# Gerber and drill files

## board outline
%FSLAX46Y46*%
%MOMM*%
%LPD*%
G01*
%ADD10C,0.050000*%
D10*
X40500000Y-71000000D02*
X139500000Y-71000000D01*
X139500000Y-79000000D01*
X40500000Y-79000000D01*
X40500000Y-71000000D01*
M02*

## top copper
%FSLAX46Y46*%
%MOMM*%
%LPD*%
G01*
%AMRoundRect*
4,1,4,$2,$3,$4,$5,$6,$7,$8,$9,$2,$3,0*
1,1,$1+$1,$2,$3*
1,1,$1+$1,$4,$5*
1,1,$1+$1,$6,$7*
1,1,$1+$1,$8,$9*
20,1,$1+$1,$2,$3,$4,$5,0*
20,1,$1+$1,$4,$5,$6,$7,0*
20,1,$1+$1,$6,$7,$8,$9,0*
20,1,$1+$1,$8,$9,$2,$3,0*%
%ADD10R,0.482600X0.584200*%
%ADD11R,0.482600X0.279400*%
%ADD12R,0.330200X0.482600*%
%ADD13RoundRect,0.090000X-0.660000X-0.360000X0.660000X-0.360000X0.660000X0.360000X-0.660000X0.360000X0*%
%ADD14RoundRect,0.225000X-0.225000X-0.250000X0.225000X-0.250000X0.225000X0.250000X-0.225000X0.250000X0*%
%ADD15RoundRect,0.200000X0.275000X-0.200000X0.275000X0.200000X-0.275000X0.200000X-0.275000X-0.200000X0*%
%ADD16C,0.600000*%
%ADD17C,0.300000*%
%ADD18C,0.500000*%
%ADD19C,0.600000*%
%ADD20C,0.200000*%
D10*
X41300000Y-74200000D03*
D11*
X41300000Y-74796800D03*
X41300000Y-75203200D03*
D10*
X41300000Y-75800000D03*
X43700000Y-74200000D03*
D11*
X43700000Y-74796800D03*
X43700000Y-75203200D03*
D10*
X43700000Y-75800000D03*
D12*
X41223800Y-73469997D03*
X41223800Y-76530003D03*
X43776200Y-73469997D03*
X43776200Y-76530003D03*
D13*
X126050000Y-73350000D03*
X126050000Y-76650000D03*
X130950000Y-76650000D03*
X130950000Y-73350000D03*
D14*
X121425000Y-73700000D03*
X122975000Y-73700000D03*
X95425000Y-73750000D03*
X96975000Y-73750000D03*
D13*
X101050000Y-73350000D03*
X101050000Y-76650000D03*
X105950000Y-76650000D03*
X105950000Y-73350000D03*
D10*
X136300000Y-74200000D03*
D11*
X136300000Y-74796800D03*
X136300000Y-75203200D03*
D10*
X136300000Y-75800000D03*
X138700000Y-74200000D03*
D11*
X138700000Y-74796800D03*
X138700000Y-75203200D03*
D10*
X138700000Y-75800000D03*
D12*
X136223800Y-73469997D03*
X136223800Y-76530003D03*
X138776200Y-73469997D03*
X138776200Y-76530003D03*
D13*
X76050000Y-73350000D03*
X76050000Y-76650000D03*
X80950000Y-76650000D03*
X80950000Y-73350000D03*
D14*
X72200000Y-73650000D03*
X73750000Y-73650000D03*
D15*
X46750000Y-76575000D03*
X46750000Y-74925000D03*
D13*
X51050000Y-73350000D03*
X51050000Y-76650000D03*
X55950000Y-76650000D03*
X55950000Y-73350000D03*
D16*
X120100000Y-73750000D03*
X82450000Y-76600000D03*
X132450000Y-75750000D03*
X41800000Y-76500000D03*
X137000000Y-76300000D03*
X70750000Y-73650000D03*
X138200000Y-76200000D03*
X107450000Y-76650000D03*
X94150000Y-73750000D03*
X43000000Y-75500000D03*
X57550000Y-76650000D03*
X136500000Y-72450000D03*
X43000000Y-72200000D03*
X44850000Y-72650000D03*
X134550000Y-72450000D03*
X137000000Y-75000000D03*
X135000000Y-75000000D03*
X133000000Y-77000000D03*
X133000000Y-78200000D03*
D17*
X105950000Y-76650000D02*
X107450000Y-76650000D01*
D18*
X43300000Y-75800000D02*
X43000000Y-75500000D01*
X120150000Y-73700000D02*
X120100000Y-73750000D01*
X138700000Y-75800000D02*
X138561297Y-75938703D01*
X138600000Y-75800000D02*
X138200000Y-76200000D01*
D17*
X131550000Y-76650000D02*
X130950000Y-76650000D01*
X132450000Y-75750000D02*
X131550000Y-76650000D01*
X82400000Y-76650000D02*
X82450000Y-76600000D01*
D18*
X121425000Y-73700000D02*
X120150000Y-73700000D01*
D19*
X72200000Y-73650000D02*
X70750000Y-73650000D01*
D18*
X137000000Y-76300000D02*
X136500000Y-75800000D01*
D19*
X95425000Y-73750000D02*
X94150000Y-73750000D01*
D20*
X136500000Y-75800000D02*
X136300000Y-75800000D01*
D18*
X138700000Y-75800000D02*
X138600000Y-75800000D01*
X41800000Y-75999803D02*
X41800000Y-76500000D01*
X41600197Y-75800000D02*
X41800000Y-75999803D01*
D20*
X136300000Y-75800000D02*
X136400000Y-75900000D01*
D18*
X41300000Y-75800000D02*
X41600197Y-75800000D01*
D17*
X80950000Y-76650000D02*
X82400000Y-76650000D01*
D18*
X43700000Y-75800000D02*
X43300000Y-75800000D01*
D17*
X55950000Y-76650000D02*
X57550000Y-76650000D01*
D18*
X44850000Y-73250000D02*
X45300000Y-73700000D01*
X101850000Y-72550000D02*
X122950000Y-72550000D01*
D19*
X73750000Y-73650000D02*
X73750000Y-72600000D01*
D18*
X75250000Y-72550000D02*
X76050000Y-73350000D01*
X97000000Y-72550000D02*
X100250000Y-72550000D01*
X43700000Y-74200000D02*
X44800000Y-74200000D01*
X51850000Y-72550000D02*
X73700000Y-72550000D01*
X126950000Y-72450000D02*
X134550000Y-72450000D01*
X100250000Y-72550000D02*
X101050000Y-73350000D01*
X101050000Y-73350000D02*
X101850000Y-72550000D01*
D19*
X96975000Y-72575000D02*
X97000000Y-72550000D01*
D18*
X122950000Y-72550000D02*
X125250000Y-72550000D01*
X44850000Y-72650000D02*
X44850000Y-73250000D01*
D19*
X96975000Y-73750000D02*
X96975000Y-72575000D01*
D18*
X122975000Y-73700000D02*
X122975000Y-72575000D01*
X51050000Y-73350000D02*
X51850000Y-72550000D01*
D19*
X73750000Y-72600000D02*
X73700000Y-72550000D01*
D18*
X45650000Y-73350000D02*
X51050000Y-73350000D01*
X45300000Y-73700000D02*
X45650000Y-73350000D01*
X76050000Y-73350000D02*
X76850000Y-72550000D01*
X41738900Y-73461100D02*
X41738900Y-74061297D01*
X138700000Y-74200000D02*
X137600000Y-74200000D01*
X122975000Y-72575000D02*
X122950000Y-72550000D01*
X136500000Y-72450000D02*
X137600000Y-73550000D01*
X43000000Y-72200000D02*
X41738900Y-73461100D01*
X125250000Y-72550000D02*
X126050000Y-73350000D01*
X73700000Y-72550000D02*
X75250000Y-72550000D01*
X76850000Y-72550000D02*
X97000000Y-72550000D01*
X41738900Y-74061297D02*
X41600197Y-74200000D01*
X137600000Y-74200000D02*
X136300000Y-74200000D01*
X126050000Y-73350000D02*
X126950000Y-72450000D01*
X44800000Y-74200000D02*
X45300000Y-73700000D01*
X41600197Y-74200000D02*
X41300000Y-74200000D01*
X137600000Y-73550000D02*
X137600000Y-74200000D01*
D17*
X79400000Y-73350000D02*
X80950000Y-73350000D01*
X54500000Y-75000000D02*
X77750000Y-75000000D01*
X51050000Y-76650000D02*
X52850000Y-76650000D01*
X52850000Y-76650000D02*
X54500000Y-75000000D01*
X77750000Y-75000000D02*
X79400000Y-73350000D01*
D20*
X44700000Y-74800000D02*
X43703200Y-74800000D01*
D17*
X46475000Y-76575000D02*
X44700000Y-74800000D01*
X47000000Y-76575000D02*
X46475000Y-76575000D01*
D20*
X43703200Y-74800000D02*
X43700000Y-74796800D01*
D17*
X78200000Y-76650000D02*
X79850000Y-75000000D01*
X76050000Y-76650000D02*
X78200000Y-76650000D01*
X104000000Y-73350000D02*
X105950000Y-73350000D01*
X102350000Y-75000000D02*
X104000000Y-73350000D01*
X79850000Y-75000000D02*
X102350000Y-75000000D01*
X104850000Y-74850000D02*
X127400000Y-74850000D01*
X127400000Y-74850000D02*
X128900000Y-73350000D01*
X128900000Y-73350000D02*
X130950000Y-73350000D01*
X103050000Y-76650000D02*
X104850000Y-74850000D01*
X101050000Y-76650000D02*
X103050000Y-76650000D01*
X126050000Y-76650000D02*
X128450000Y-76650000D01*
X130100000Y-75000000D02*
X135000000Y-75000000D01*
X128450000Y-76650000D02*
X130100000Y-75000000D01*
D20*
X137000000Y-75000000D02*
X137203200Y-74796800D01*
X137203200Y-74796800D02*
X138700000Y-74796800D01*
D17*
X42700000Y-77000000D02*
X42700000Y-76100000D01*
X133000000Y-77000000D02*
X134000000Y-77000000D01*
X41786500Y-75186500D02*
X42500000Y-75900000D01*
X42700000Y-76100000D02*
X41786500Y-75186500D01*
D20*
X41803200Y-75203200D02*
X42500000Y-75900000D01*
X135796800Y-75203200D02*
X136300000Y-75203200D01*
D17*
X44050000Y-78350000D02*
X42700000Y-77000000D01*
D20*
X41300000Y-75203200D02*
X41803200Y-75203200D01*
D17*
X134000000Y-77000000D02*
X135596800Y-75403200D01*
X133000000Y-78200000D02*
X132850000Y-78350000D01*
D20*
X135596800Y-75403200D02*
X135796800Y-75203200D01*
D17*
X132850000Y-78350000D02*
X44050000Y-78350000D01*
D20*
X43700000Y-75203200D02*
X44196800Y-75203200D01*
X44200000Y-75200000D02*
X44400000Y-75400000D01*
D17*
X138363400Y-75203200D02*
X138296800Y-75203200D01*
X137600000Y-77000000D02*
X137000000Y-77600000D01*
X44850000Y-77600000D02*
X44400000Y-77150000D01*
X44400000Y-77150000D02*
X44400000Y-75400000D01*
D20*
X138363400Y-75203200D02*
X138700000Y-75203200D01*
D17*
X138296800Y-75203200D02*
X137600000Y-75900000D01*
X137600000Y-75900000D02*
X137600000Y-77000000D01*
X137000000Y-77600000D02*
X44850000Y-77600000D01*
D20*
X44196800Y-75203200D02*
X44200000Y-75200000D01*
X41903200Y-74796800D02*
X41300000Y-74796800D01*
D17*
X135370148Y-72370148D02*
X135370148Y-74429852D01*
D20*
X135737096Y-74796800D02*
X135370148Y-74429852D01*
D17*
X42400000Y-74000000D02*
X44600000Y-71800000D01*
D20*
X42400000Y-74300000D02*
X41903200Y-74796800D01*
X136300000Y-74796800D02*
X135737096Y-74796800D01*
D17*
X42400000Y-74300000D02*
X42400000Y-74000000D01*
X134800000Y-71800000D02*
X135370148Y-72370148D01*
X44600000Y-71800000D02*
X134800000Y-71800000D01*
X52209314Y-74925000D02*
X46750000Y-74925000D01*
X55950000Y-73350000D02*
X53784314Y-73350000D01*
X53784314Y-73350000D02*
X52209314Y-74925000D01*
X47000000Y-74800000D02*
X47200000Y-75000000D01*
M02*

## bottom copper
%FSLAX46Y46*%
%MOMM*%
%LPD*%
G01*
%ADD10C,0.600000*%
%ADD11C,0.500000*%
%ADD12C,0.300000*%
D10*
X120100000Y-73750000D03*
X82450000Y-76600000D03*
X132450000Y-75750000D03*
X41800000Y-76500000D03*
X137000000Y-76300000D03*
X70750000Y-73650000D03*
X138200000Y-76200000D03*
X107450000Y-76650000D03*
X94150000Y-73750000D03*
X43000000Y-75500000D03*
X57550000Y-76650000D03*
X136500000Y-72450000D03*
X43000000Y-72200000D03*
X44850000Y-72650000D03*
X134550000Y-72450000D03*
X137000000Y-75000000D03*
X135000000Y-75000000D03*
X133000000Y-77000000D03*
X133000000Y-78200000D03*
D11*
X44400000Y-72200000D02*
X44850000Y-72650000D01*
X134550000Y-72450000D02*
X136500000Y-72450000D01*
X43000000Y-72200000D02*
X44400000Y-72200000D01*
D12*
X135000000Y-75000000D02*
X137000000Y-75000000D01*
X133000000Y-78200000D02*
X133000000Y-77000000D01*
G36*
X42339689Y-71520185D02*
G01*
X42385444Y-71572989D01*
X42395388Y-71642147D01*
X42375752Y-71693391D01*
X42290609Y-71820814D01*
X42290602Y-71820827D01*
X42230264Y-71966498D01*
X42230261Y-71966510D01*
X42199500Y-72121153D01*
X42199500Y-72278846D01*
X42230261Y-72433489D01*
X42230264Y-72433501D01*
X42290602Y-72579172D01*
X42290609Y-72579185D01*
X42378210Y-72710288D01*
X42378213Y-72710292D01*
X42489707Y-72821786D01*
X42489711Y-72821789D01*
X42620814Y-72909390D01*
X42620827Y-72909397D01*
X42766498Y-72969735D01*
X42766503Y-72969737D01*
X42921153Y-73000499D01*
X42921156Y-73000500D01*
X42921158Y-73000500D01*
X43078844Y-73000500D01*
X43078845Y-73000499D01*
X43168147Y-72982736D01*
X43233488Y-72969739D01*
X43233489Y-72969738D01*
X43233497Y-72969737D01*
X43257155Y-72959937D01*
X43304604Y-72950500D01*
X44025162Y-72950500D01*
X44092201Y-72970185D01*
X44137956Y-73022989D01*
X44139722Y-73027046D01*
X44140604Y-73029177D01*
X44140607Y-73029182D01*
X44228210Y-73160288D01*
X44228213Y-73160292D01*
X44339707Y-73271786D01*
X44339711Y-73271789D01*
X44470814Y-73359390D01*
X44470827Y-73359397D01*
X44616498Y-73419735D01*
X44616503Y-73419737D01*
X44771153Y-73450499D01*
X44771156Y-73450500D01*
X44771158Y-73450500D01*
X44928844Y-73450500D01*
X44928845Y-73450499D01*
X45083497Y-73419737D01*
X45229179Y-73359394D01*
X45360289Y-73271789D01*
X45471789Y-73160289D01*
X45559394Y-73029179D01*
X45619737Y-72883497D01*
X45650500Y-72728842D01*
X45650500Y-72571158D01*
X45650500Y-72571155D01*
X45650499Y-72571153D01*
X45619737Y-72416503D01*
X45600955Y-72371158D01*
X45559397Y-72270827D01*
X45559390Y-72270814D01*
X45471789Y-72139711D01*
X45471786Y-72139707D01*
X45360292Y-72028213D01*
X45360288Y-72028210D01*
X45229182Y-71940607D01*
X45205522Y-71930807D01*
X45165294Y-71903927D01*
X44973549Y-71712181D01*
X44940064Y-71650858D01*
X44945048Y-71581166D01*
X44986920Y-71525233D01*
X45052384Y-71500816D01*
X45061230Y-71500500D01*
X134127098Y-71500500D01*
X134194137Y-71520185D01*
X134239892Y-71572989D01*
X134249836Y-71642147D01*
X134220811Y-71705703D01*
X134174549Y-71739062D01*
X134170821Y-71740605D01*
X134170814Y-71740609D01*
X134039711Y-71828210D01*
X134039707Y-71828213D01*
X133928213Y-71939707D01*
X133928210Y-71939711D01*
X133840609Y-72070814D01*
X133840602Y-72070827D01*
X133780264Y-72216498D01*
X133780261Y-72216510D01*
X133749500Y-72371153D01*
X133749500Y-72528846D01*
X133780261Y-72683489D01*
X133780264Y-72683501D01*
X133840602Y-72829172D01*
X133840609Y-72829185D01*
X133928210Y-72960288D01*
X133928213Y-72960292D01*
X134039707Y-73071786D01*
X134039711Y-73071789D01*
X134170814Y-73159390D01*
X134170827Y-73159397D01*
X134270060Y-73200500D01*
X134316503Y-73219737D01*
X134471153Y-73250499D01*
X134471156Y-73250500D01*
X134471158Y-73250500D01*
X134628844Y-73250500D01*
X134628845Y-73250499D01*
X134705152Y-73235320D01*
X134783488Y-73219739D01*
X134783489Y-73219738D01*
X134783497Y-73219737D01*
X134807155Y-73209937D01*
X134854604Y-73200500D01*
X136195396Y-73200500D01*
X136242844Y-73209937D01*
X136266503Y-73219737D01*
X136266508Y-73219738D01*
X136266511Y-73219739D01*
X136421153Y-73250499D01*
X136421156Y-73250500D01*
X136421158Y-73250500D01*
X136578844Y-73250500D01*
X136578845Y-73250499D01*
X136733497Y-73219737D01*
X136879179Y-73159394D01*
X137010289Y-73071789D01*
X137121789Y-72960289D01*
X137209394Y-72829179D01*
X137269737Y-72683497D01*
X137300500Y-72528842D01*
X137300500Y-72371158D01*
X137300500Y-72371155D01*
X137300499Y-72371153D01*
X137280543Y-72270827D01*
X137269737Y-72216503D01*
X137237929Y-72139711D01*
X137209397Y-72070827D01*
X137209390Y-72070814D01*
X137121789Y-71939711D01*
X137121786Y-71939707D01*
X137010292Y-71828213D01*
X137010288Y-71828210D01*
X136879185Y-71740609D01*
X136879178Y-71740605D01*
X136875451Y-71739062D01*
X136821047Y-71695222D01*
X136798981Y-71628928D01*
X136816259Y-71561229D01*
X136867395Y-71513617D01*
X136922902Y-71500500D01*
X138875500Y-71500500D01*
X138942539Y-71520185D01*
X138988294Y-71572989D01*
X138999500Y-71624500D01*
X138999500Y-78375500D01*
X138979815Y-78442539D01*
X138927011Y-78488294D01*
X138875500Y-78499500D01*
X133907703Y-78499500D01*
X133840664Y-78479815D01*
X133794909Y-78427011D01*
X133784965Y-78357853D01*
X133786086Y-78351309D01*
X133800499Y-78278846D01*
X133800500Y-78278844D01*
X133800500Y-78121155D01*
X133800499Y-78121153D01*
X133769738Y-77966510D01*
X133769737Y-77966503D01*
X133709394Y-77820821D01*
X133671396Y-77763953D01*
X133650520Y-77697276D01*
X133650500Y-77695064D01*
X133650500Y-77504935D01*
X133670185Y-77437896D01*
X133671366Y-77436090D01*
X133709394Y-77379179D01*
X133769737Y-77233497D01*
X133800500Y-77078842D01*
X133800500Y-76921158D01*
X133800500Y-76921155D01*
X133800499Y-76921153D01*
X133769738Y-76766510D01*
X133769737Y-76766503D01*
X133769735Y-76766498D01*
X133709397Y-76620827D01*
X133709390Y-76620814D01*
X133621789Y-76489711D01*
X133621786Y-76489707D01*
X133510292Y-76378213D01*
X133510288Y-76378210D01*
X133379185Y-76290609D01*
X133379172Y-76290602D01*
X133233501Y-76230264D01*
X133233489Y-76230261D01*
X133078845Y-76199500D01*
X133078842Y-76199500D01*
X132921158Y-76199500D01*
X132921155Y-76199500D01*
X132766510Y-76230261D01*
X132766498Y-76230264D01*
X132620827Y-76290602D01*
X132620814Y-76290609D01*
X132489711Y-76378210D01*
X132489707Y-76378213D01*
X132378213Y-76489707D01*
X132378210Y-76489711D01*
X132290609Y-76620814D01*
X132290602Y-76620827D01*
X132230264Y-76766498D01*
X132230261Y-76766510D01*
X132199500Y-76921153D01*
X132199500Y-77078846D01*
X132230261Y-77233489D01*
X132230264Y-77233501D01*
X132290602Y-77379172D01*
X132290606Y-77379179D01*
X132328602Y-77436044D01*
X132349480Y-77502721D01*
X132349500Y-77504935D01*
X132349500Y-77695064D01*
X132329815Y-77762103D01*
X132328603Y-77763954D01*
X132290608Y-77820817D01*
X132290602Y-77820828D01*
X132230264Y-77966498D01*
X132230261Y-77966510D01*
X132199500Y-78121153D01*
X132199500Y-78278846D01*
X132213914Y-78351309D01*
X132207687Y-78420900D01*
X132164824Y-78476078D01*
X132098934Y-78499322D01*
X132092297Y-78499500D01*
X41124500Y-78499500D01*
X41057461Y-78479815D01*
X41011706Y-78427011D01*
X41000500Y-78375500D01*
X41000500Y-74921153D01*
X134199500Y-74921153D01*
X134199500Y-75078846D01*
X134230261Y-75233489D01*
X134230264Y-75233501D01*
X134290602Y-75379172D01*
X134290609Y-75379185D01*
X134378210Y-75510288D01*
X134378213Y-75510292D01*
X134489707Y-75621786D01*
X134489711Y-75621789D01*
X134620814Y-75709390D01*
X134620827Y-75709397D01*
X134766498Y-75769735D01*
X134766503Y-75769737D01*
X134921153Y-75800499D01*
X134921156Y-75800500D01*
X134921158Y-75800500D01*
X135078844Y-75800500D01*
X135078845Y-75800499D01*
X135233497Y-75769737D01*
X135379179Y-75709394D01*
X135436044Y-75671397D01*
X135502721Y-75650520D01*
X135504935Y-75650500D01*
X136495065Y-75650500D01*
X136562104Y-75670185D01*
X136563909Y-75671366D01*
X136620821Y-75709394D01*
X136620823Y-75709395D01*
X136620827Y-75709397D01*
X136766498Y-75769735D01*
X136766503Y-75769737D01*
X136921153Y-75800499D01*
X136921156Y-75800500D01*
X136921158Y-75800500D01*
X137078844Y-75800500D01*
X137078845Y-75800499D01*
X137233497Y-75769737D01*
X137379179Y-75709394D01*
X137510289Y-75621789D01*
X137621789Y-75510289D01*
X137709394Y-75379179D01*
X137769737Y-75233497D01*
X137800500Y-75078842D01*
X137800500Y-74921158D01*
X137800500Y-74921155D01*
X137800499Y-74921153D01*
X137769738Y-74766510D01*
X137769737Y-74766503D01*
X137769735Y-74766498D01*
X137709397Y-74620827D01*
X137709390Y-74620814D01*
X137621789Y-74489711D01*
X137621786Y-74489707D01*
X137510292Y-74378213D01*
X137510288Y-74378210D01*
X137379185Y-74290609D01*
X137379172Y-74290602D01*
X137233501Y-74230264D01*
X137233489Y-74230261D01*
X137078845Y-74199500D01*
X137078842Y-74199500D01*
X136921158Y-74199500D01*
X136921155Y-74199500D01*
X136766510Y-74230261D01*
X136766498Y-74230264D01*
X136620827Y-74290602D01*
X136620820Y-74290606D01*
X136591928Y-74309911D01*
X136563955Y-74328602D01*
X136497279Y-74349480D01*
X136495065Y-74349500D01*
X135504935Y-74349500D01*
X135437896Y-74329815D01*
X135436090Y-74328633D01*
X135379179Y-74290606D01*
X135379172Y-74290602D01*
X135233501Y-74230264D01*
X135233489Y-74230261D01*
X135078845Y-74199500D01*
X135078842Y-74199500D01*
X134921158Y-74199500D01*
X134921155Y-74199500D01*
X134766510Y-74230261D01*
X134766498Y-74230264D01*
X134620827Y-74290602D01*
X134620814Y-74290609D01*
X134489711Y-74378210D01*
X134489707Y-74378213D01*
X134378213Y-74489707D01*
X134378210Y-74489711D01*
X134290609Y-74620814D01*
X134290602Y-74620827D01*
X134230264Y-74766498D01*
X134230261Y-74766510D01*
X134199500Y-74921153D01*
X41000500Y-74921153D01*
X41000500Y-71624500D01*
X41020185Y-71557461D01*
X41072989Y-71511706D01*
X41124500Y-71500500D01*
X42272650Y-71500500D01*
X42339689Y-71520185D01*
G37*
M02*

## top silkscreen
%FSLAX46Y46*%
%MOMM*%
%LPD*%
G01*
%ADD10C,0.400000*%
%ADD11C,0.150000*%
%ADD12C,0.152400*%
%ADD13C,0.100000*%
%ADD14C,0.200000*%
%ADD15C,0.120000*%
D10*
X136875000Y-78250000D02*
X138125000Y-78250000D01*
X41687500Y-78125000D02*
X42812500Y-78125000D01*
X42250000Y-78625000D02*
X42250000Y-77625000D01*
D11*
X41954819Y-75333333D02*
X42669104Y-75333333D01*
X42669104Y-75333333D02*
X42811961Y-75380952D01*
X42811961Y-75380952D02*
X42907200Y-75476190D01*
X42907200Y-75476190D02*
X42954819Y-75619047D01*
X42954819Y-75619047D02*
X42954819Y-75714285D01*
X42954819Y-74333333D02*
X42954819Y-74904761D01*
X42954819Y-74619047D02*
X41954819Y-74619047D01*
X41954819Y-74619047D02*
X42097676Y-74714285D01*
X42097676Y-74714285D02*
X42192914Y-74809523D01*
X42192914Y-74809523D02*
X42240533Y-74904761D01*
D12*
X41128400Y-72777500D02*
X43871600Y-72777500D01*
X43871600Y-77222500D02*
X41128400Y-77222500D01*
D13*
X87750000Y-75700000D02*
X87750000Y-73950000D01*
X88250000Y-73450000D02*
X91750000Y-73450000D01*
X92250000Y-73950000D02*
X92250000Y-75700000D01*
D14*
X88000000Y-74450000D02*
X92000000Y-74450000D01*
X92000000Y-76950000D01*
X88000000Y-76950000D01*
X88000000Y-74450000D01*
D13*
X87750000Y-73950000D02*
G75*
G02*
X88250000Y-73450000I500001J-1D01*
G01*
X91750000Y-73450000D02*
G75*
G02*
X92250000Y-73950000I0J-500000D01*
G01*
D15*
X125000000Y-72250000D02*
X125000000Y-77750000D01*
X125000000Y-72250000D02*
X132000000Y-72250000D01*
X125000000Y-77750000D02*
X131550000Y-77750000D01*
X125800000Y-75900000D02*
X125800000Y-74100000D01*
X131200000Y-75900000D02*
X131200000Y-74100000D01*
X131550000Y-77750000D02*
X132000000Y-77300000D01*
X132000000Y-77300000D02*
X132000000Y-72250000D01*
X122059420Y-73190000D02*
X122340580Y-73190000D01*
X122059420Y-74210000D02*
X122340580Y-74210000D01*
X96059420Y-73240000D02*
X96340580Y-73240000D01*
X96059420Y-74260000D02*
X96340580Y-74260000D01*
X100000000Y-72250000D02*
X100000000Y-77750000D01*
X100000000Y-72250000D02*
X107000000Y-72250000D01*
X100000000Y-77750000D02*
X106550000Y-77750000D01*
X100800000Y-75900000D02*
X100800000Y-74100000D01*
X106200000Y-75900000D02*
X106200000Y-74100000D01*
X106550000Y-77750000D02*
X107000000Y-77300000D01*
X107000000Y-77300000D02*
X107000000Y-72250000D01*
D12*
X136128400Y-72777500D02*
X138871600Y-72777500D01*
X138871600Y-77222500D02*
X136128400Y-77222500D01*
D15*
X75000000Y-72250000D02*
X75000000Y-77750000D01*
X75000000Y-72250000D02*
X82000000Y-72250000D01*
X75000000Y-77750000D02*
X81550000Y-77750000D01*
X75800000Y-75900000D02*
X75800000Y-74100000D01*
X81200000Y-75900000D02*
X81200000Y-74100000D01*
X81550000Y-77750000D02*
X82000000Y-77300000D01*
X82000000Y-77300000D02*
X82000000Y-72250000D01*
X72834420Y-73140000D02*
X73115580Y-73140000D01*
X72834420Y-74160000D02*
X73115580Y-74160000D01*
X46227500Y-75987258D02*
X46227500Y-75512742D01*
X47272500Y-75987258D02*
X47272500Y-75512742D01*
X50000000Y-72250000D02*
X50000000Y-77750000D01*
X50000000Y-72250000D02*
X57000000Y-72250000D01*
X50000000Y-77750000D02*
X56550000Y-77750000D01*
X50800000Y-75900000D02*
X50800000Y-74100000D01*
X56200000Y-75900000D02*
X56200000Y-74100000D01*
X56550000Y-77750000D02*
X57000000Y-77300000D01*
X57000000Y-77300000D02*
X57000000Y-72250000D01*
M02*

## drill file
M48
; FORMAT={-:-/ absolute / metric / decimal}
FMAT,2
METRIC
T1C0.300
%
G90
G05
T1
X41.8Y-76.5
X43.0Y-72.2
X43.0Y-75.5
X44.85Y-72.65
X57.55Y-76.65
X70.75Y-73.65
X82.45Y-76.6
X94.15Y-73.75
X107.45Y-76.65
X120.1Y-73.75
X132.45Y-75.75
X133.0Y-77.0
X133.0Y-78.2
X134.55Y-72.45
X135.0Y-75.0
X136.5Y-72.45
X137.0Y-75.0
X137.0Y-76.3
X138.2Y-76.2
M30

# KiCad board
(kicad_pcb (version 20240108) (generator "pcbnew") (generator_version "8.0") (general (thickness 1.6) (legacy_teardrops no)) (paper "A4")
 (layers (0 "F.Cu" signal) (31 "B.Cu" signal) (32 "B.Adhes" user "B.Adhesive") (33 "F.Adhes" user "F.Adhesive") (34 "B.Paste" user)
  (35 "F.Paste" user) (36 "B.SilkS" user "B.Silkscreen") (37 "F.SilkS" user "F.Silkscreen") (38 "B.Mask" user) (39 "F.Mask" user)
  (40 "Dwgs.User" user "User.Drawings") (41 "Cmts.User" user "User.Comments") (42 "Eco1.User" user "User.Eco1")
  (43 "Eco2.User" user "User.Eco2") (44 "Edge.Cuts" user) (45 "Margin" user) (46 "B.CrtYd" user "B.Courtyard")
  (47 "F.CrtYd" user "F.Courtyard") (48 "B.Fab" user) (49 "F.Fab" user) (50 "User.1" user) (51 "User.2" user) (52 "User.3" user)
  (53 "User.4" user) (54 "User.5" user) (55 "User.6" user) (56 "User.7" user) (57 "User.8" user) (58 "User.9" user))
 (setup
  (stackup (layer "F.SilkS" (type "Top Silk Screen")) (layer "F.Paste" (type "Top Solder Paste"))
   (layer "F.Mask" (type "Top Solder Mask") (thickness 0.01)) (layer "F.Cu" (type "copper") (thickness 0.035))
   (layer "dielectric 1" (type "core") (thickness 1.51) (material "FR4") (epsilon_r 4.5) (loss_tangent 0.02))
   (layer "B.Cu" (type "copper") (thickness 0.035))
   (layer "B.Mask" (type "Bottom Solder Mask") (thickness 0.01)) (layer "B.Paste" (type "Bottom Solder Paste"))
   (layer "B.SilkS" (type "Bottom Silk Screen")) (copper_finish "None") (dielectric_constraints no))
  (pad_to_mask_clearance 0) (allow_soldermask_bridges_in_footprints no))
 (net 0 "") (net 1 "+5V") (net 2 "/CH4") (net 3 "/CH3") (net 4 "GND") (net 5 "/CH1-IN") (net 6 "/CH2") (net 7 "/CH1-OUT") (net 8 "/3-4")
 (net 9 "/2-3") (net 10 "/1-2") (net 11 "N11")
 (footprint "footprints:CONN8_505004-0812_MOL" (layer "F.Cu") (at 42.5 75 90)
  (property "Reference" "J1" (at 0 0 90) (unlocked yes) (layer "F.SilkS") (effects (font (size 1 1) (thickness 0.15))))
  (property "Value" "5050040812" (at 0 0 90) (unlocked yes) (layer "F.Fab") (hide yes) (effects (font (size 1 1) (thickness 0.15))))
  (fp_line (start 2.2225 -1.3716) (end 2.2225 1.3716) (stroke (width 0.1524) (type solid)) (layer "F.SilkS"))
  (fp_line (start -2.2225 1.3716) (end -2.2225 -1.3716) (stroke (width 0.1524) (type solid)) (layer "F.SilkS"))
  (pad "1" smd rect (at 0.8 -1.2 90) (size 0.5842 0.4826) (layers "F.Cu" "F.Paste" "F.Mask") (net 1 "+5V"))
  (pad "2" smd rect (at 0.2032 -1.2 90) (size 0.2794 0.4826) (layers "F.Cu" "F.Paste" "F.Mask") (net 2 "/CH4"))
  (pad "3" smd rect (at -0.2032 -1.2 90) (size 0.2794 0.4826) (layers "F.Cu" "F.Paste" "F.Mask") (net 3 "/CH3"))
  (pad "4" smd rect (at -0.8 -1.2 90) (size 0.5842 0.4826) (layers "F.Cu" "F.Paste" "F.Mask") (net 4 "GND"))
  (pad "5" smd rect (at 0.8 1.2 90) (size 0.5842 0.4826) (layers "F.Cu" "F.Paste" "F.Mask") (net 1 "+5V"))
  (pad "6" smd rect (at 0.2032 1.2 90) (size 0.2794 0.4826) (layers "F.Cu" "F.Paste" "F.Mask") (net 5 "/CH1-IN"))
  (pad "7" smd rect (at -0.2032 1.2 90) (size 0.2794 0.4826) (layers "F.Cu" "F.Paste" "F.Mask") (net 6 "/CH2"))
  (pad "8" smd rect (at -0.8 1.2 90) (size 0.5842 0.4826) (layers "F.Cu" "F.Paste" "F.Mask") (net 4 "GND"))
  (pad "9" smd rect (at 1.530003 -1.2762 90) (size 0.4826 0.3302) (layers "F.Cu" "F.Paste" "F.Mask"))
  (pad "10" smd rect (at -1.530003 -1.2762 90) (size 0.4826 0.3302) (layers "F.Cu" "F.Paste" "F.Mask"))
  (pad "11" smd rect (at 1.530003 1.2762 90) (size 0.4826 0.3302) (layers "F.Cu" "F.Paste" "F.Mask"))
  (pad "12" smd rect (at -1.530003 1.2762 90) (size 0.4826 0.3302) (layers "F.Cu" "F.Paste" "F.Mask")))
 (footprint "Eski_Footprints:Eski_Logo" (layer "F.Cu") (at 90 76.95)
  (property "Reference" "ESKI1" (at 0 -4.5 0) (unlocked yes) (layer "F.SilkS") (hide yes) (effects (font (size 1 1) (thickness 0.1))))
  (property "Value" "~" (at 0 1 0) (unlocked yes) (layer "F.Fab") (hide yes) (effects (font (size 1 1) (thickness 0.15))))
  (fp_line (start -2.25 -1.25) (end -2.25 -3) (stroke (width 0.1) (type default)) (layer "F.SilkS"))
  (fp_line (start -1.75 -3.5) (end 1.75 -3.5) (stroke (width 0.1) (type default)) (layer "F.SilkS"))
  (fp_line (start 2.25 -3) (end 2.25 -1.25) (stroke (width 0.1) (type default)) (layer "F.SilkS"))
  (fp_rect (start -2 -2.5) (end 2 0) (stroke (width 0.2) (type default)) (fill none) (layer "F.SilkS"))
  (fp_arc (start -2.25 -3) (mid -2.103553 -3.353553) (end -1.75 -3.5) (stroke (width 0.1) (type default)) (layer "F.SilkS"))
  (fp_arc (start 1.75 -3.5) (mid 2.103553 -3.353553) (end 2.25 -3) (stroke (width 0.1) (type default)) (layer "F.SilkS")))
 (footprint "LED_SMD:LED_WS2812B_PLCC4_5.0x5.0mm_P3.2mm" (layer "F.Cu") (at 128.5 75)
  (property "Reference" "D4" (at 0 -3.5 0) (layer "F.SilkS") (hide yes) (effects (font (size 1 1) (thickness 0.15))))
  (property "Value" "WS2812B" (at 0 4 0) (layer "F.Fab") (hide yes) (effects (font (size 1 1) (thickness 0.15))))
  (fp_line (start -3.5 -2.75) (end -3.5 2.75) (stroke (width 0.12) (type default)) (layer "F.SilkS"))
  (fp_line (start -3.5 -2.75) (end 3.5 -2.75) (stroke (width 0.12) (type solid)) (layer "F.SilkS"))
  (fp_line (start -3.5 2.75) (end 3.05 2.75) (stroke (width 0.12) (type solid)) (layer "F.SilkS"))
  (fp_line (start -2.7 0.9) (end -2.7 -0.9) (stroke (width 0.12) (type default)) (layer "F.SilkS"))
  (fp_line (start 2.7 0.9) (end 2.7 -0.9) (stroke (width 0.12) (type default)) (layer "F.SilkS"))
  (fp_line (start 3.05 2.75) (end 3.5 2.3) (stroke (width 0.12) (type default)) (layer "F.SilkS"))
  (fp_line (start 3.5 2.3) (end 3.5 -2.75) (stroke (width 0.12) (type default)) (layer "F.SilkS"))
  (pad "1" smd roundrect (at -2.45 -1.65) (size 1.5 0.9) (layers "F.Cu" "F.Paste" "F.Mask") (roundrect_rratio 0.1) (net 1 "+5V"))
  (pad "2" smd roundrect (at -2.45 1.65) (size 1.5 0.9) (layers "F.Cu" "F.Paste" "F.Mask") (roundrect_rratio 0.1) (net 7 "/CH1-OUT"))
  (pad "3" smd roundrect (at 2.45 1.65) (size 1.5 0.9) (layers "F.Cu" "F.Paste" "F.Mask") (roundrect_rratio 0.1) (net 4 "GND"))
  (pad "4" smd roundrect (at 2.45 -1.65) (size 1.5 0.9) (layers "F.Cu" "F.Paste" "F.Mask") (roundrect_rratio 0.1) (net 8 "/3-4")))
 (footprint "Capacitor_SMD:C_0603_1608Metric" (layer "F.Cu") (at 122.2 73.7)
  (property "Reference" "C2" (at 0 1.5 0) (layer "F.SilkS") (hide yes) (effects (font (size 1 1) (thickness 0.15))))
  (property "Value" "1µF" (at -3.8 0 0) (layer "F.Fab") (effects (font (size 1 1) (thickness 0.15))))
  (fp_line (start -0.14058 -0.51) (end 0.14058 -0.51) (stroke (width 0.12) (type solid)) (layer "F.SilkS"))
  (fp_line (start -0.14058 0.51) (end 0.14058 0.51) (stroke (width 0.12) (type solid)) (layer "F.SilkS"))
  (pad "1" smd roundrect (at -0.775 0) (size 0.9 0.95) (layers "F.Cu" "F.Paste" "F.Mask") (roundrect_rratio 0.25) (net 4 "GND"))
  (pad "2" smd roundrect (at 0.775 0) (size 0.9 0.95) (layers "F.Cu" "F.Paste" "F.Mask") (roundrect_rratio 0.25) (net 1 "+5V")))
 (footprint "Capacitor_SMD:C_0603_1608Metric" (layer "F.Cu") (at 96.2 73.75)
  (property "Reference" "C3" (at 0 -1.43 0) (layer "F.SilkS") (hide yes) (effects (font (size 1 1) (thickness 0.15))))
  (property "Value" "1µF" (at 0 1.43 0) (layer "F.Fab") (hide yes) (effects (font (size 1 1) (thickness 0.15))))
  (fp_line (start -0.14058 -0.51) (end 0.14058 -0.51) (stroke (width 0.12) (type solid)) (layer "F.SilkS"))
  (fp_line (start -0.14058 0.51) (end 0.14058 0.51) (stroke (width 0.12) (type solid)) (layer "F.SilkS"))
  (pad "1" smd roundrect (at -0.775 0) (size 0.9 0.95) (layers "F.Cu" "F.Paste" "F.Mask") (roundrect_rratio 0.25) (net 4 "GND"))
  (pad "2" smd roundrect (at 0.775 0) (size 0.9 0.95) (layers "F.Cu" "F.Paste" "F.Mask") (roundrect_rratio 0.25) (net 1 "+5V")))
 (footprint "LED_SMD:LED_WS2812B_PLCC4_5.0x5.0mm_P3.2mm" (layer "F.Cu") (at 103.5 75)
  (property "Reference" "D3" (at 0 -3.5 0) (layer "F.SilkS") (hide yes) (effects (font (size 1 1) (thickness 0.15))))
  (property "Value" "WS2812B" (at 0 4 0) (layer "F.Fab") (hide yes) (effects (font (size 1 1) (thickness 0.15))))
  (fp_line (start -3.5 -2.75) (end -3.5 2.75) (stroke (width 0.12) (type default)) (layer "F.SilkS"))
  (fp_line (start -3.5 -2.75) (end 3.5 -2.75) (stroke (width 0.12) (type solid)) (layer "F.SilkS"))
  (fp_line (start -3.5 2.75) (end 3.05 2.75) (stroke (width 0.12) (type solid)) (layer "F.SilkS"))
  (fp_line (start -2.7 0.9) (end -2.7 -0.9) (stroke (width 0.12) (type default)) (layer "F.SilkS"))
  (fp_line (start 2.7 0.9) (end 2.7 -0.9) (stroke (width 0.12) (type default)) (layer "F.SilkS"))
  (fp_line (start 3.05 2.75) (end 3.5 2.3) (stroke (width 0.12) (type default)) (layer "F.SilkS"))
  (fp_line (start 3.5 2.3) (end 3.5 -2.75) (stroke (width 0.12) (type default)) (layer "F.SilkS"))
  (pad "1" smd roundrect (at -2.45 -1.65) (size 1.5 0.9) (layers "F.Cu" "F.Paste" "F.Mask") (roundrect_rratio 0.1) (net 1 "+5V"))
  (pad "2" smd roundrect (at -2.45 1.65) (size 1.5 0.9) (layers "F.Cu" "F.Paste" "F.Mask") (roundrect_rratio 0.1) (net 8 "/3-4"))
  (pad "3" smd roundrect (at 2.45 1.65) (size 1.5 0.9) (layers "F.Cu" "F.Paste" "F.Mask") (roundrect_rratio 0.1) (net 4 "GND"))
  (pad "4" smd roundrect (at 2.45 -1.65) (size 1.5 0.9) (layers "F.Cu" "F.Paste" "F.Mask") (roundrect_rratio 0.1) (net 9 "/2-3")))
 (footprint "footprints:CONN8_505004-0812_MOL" (layer "F.Cu") (at 137.5 75 90)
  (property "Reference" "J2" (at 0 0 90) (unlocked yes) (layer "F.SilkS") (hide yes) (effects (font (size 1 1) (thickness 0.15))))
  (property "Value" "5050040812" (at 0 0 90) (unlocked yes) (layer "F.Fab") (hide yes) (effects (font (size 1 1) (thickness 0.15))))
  (fp_line (start 2.2225 -1.3716) (end 2.2225 1.3716) (stroke (width 0.1524) (type solid)) (layer "F.SilkS"))
  (fp_line (start -2.2225 1.3716) (end -2.2225 -1.3716) (stroke (width 0.1524) (type solid)) (layer "F.SilkS"))
  (pad "1" smd rect (at 0.8 -1.2 90) (size 0.5842 0.4826) (layers "F.Cu" "F.Paste" "F.Mask") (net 1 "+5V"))
  (pad "2" smd rect (at 0.2032 -1.2 90) (size 0.2794 0.4826) (layers "F.Cu" "F.Paste" "F.Mask") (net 2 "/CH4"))
  (pad "3" smd rect (at -0.2032 -1.2 90) (size 0.2794 0.4826) (layers "F.Cu" "F.Paste" "F.Mask") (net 3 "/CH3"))
  (pad "4" smd rect (at -0.8 -1.2 90) (size 0.5842 0.4826) (layers "F.Cu" "F.Paste" "F.Mask") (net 4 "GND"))
  (pad "5" smd rect (at 0.8 1.2 90) (size 0.5842 0.4826) (layers "F.Cu" "F.Paste" "F.Mask") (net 1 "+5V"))
  (pad "6" smd rect (at 0.2032 1.2 90) (size 0.2794 0.4826) (layers "F.Cu" "F.Paste" "F.Mask") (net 7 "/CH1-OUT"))
  (pad "7" smd rect (at -0.2032 1.2 90) (size 0.2794 0.4826) (layers "F.Cu" "F.Paste" "F.Mask") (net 6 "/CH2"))
  (pad "8" smd rect (at -0.8 1.2 90) (size 0.5842 0.4826) (layers "F.Cu" "F.Paste" "F.Mask") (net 4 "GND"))
  (pad "9" smd rect (at 1.530003 -1.2762 90) (size 0.4826 0.3302) (layers "F.Cu" "F.Paste" "F.Mask"))
  (pad "10" smd rect (at -1.530003 -1.2762 90) (size 0.4826 0.3302) (layers "F.Cu" "F.Paste" "F.Mask"))
  (pad "11" smd rect (at 1.530003 1.2762 90) (size 0.4826 0.3302) (layers "F.Cu" "F.Paste" "F.Mask"))
  (pad "12" smd rect (at -1.530003 1.2762 90) (size 0.4826 0.3302) (layers "F.Cu" "F.Paste" "F.Mask")))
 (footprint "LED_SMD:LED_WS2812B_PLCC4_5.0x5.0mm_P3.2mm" (layer "F.Cu") (at 78.5 75)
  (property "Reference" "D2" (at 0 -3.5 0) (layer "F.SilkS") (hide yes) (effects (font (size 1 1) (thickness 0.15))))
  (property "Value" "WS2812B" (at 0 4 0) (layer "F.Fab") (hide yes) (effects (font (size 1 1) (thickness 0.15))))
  (fp_line (start -3.5 -2.75) (end -3.5 2.75) (stroke (width 0.12) (type default)) (layer "F.SilkS"))
  (fp_line (start -3.5 -2.75) (end 3.5 -2.75) (stroke (width 0.12) (type solid)) (layer "F.SilkS"))
  (fp_line (start -3.5 2.75) (end 3.05 2.75) (stroke (width 0.12) (type solid)) (layer "F.SilkS"))
  (fp_line (start -2.7 0.9) (end -2.7 -0.9) (stroke (width 0.12) (type default)) (layer "F.SilkS"))
  (fp_line (start 2.7 0.9) (end 2.7 -0.9) (stroke (width 0.12) (type default)) (layer "F.SilkS"))
  (fp_line (start 3.05 2.75) (end 3.5 2.3) (stroke (width 0.12) (type default)) (layer "F.SilkS"))
  (fp_line (start 3.5 2.3) (end 3.5 -2.75) (stroke (width 0.12) (type default)) (layer "F.SilkS"))
  (pad "1" smd roundrect (at -2.45 -1.65) (size 1.5 0.9) (layers "F.Cu" "F.Paste" "F.Mask") (roundrect_rratio 0.1) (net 1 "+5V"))
  (pad "2" smd roundrect (at -2.45 1.65) (size 1.5 0.9) (layers "F.Cu" "F.Paste" "F.Mask") (roundrect_rratio 0.1) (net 9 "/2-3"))
  (pad "3" smd roundrect (at 2.45 1.65) (size 1.5 0.9) (layers "F.Cu" "F.Paste" "F.Mask") (roundrect_rratio 0.1) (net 4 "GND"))
  (pad "4" smd roundrect (at 2.45 -1.65) (size 1.5 0.9) (layers "F.Cu" "F.Paste" "F.Mask") (roundrect_rratio 0.1) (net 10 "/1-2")))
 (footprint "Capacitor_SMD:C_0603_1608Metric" (layer "F.Cu") (at 72.975 73.65)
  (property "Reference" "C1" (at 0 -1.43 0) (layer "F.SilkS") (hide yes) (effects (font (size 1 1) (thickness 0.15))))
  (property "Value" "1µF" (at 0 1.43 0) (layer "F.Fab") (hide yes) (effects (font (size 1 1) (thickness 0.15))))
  (fp_line (start -0.14058 -0.51) (end 0.14058 -0.51) (stroke (width 0.12) (type solid)) (layer "F.SilkS"))
  (fp_line (start -0.14058 0.51) (end 0.14058 0.51) (stroke (width 0.12) (type solid)) (layer "F.SilkS"))
  (pad "1" smd roundrect (at -0.775 0) (size 0.9 0.95) (layers "F.Cu" "F.Paste" "F.Mask") (roundrect_rratio 0.25) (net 4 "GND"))
  (pad "2" smd roundrect (at 0.775 0) (size 0.9 0.95) (layers "F.Cu" "F.Paste" "F.Mask") (roundrect_rratio 0.25) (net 1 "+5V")))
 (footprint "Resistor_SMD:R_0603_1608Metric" (layer "F.Cu") (at 46.75 75.75 90)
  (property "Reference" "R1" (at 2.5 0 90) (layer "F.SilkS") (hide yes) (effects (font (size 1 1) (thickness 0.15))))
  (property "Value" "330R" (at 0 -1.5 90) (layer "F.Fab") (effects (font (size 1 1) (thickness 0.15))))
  (fp_line (start -0.237258 -0.5225) (end 0.237258 -0.5225) (stroke (width 0.12) (type solid)) (layer "F.SilkS"))
  (fp_line (start -0.237258 0.5225) (end 0.237258 0.5225) (stroke (width 0.12) (type solid)) (layer "F.SilkS"))
  (pad "1" smd roundrect (at -0.825 0 90) (size 0.8 0.95) (layers "F.Cu" "F.Paste" "F.Mask") (roundrect_rratio 0.25) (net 5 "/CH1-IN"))
  (pad "2" smd roundrect (at 0.825 0 90) (size 0.8 0.95) (layers "F.Cu" "F.Paste" "F.Mask") (roundrect_rratio 0.25) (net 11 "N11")))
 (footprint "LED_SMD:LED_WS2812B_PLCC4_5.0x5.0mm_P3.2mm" (layer "F.Cu") (at 53.5 75)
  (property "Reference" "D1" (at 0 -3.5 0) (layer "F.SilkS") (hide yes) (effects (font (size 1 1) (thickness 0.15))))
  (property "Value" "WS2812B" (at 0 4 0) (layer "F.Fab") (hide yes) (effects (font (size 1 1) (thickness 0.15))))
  (fp_line (start -3.5 -2.75) (end -3.5 2.75) (stroke (width 0.12) (type default)) (layer "F.SilkS"))
  (fp_line (start -3.5 -2.75) (end 3.5 -2.75) (stroke (width 0.12) (type solid)) (layer "F.SilkS"))
  (fp_line (start -3.5 2.75) (end 3.05 2.75) (stroke (width 0.12) (type solid)) (layer "F.SilkS"))
  (fp_line (start -2.7 0.9) (end -2.7 -0.9) (stroke (width 0.12) (type default)) (layer "F.SilkS"))
  (fp_line (start 2.7 0.9) (end 2.7 -0.9) (stroke (width 0.12) (type default)) (layer "F.SilkS"))
  (fp_line (start 3.05 2.75) (end 3.5 2.3) (stroke (width 0.12) (type default)) (layer "F.SilkS"))
  (fp_line (start 3.5 2.3) (end 3.5 -2.75) (stroke (width 0.12) (type default)) (layer "F.SilkS"))
  (pad "1" smd roundrect (at -2.45 -1.65) (size 1.5 0.9) (layers "F.Cu" "F.Paste" "F.Mask") (roundrect_rratio 0.1) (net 1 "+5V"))
  (pad "2" smd roundrect (at -2.45 1.65) (size 1.5 0.9) (layers "F.Cu" "F.Paste" "F.Mask") (roundrect_rratio 0.1) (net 10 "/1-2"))
  (pad "3" smd roundrect (at 2.45 1.65) (size 1.5 0.9) (layers "F.Cu" "F.Paste" "F.Mask") (roundrect_rratio 0.1) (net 4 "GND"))
  (pad "4" smd roundrect (at 2.45 -1.65) (size 1.5 0.9) (layers "F.Cu" "F.Paste" "F.Mask") (roundrect_rratio 0.1) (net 11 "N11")))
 (gr_line (start 136.875 78.25) (end 138.125 78.25) (stroke (width 0.4) (type default)) (layer "F.SilkS"))
 (gr_line (start 41.6875 78.125) (end 42.8125 78.125) (stroke (width 0.4) (type default)) (layer "F.SilkS"))
 (gr_line (start 42.25 78.625) (end 42.25 77.625) (stroke (width 0.4) (type default)) (layer "F.SilkS"))
 (gr_rect (start 40.5 71) (end 139.5 79) (stroke (width 0.05) (type default)) (fill none) (layer "Edge.Cuts"))
 (segment (start 105.95 76.65) (end 107.45 76.65) (width 0.3) (layer "F.Cu") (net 4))
 (segment (start 43.3 75.8) (end 43 75.5) (width 0.5) (layer "F.Cu") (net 4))
 (segment (start 120.15 73.7) (end 120.1 73.75) (width 0.5) (layer "F.Cu") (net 4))
 (segment (start 138.7 75.8) (end 138.561297 75.938703) (width 0.5) (layer "F.Cu") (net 4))
 (segment (start 138.6 75.8) (end 138.2 76.2) (width 0.5) (layer "F.Cu") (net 4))
 (segment (start 131.55 76.65) (end 130.95 76.65) (width 0.3) (layer "F.Cu") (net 4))
 (segment (start 132.45 75.75) (end 131.55 76.65) (width 0.3) (layer "F.Cu") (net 4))
 (segment (start 82.4 76.65) (end 82.45 76.6) (width 0.3) (layer "F.Cu") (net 4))
 (segment (start 121.425 73.7) (end 120.15 73.7) (width 0.5) (layer "F.Cu") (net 4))
 (segment (start 72.2 73.65) (end 70.75 73.65) (width 0.6) (layer "F.Cu") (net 4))
 (segment (start 137 76.3) (end 136.5 75.8) (width 0.5) (layer "F.Cu") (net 4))
 (segment (start 95.425 73.75) (end 94.15 73.75) (width 0.6) (layer "F.Cu") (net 4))
 (segment (start 136.5 75.8) (end 136.3 75.8) (width 0.2) (layer "F.Cu") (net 4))
 (segment (start 138.7 75.8) (end 138.6 75.8) (width 0.5) (layer "F.Cu") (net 4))
 (segment (start 41.8 75.999803) (end 41.8 76.5) (width 0.5) (layer "F.Cu") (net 4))
 (segment (start 41.600197 75.8) (end 41.8 75.999803) (width 0.5) (layer "F.Cu") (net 4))
 (segment (start 136.3 75.8) (end 136.4 75.9) (width 0.2) (layer "F.Cu") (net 4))
 (segment (start 41.3 75.8) (end 41.600197 75.8) (width 0.5) (layer "F.Cu") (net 4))
 (segment (start 80.95 76.65) (end 82.4 76.65) (width 0.3) (layer "F.Cu") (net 4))
 (segment (start 43.7 75.8) (end 43.3 75.8) (width 0.5) (layer "F.Cu") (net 4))
 (segment (start 55.95 76.65) (end 57.55 76.65) (width 0.3) (layer "F.Cu") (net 4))
 (via (at 120.1 73.75) (size 0.6) (drill 0.3) (layers "F.Cu" "B.Cu") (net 4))
 (via (at 82.45 76.6) (size 0.6) (drill 0.3) (layers "F.Cu" "B.Cu") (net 4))
 (via (at 132.45 75.75) (size 0.6) (drill 0.3) (layers "F.Cu" "B.Cu") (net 4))
 (via (at 41.8 76.5) (size 0.6) (drill 0.3) (layers "F.Cu" "B.Cu") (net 4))
 (via (at 137 76.3) (size 0.6) (drill 0.3) (layers "F.Cu" "B.Cu") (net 4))
 (via (at 70.75 73.65) (size 0.6) (drill 0.3) (layers "F.Cu" "B.Cu") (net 4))
 (via (at 138.2 76.2) (size 0.6) (drill 0.3) (layers "F.Cu" "B.Cu") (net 4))
 (via (at 107.45 76.65) (size 0.6) (drill 0.3) (layers "F.Cu" "B.Cu") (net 4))
 (via (at 94.15 73.75) (size 0.6) (drill 0.3) (layers "F.Cu" "B.Cu") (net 4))
 (via (at 43 75.5) (size 0.6) (drill 0.3) (layers "F.Cu" "B.Cu") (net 4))
 (via (at 57.55 76.65) (size 0.6) (drill 0.3) (layers "F.Cu" "B.Cu") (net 4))
 (segment (start 44.85 73.25) (end 45.3 73.7) (width 0.5) (layer "F.Cu") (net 1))
 (segment (start 101.85 72.55) (end 122.95 72.55) (width 0.5) (layer "F.Cu") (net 1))
 (segment (start 73.75 73.65) (end 73.75 72.6) (width 0.6) (layer "F.Cu") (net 1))
 (segment (start 75.25 72.55) (end 76.05 73.35) (width 0.5) (layer "F.Cu") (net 1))
 (segment (start 97 72.55) (end 100.25 72.55) (width 0.5) (layer "F.Cu") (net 1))
 (segment (start 43.7 74.2) (end 44.8 74.2) (width 0.5) (layer "F.Cu") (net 1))
 (segment (start 51.85 72.55) (end 73.7 72.55) (width 0.5) (layer "F.Cu") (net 1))
 (segment (start 126.95 72.45) (end 134.55 72.45) (width 0.5) (layer "F.Cu") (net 1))
 (segment (start 100.25 72.55) (end 101.05 73.35) (width 0.5) (layer "F.Cu") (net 1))
 (segment (start 101.05 73.35) (end 101.85 72.55) (width 0.5) (layer "F.Cu") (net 1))
 (segment (start 96.975 72.575) (end 97 72.55) (width 0.6) (layer "F.Cu") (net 1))
 (segment (start 122.95 72.55) (end 125.25 72.55) (width 0.5) (layer "F.Cu") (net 1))
 (segment (start 44.85 72.65) (end 44.85 73.25) (width 0.5) (layer "F.Cu") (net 1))
 (segment (start 96.975 73.75) (end 96.975 72.575) (width 0.6) (layer "F.Cu") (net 1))
 (segment (start 122.975 73.7) (end 122.975 72.575) (width 0.5) (layer "F.Cu") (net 1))
 (segment (start 51.05 73.35) (end 51.85 72.55) (width 0.5) (layer "F.Cu") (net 1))
 (segment (start 73.75 72.6) (end 73.7 72.55) (width 0.6) (layer "F.Cu") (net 1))
 (segment (start 45.65 73.35) (end 51.05 73.35) (width 0.5) (layer "F.Cu") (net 1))
 (segment (start 45.3 73.7) (end 45.65 73.35) (width 0.5) (layer "F.Cu") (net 1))
 (segment (start 76.05 73.35) (end 76.85 72.55) (width 0.5) (layer "F.Cu") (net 1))
 (segment (start 41.7389 73.4611) (end 41.7389 74.061297) (width 0.5) (layer "F.Cu") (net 1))
 (segment (start 138.7 74.2) (end 137.6 74.2) (width 0.5) (layer "F.Cu") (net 1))
 (segment (start 122.975 72.575) (end 122.95 72.55) (width 0.5) (layer "F.Cu") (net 1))
 (segment (start 136.5 72.45) (end 137.6 73.55) (width 0.5) (layer "F.Cu") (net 1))
 (segment (start 43 72.2) (end 41.7389 73.4611) (width 0.5) (layer "F.Cu") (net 1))
 (segment (start 125.25 72.55) (end 126.05 73.35) (width 0.5) (layer "F.Cu") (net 1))
 (segment (start 73.7 72.55) (end 75.25 72.55) (width 0.5) (layer "F.Cu") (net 1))
 (segment (start 76.85 72.55) (end 97 72.55) (width 0.5) (layer "F.Cu") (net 1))
 (segment (start 41.7389 74.061297) (end 41.600197 74.2) (width 0.5) (layer "F.Cu") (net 1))
 (segment (start 137.6 74.2) (end 136.3 74.2) (width 0.5) (layer "F.Cu") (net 1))
 (segment (start 126.05 73.35) (end 126.95 72.45) (width 0.5) (layer "F.Cu") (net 1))
 (segment (start 44.8 74.2) (end 45.3 73.7) (width 0.5) (layer "F.Cu") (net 1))
 (segment (start 41.600197 74.2) (end 41.3 74.2) (width 0.5) (layer "F.Cu") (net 1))
 (segment (start 137.6 73.55) (end 137.6 74.2) (width 0.5) (layer "F.Cu") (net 1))
 (via (at 136.5 72.45) (size 0.6) (drill 0.3) (layers "F.Cu" "B.Cu") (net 1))
 (via (at 43 72.2) (size 0.6) (drill 0.3) (layers "F.Cu" "B.Cu") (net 1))
 (via (at 44.85 72.65) (size 0.6) (drill 0.3) (layers "F.Cu" "B.Cu") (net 1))
 (via (at 134.55 72.45) (size 0.6) (drill 0.3) (layers "F.Cu" "B.Cu") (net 1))
 (segment (start 44.4 72.2) (end 44.85 72.65) (width 0.5) (layer "B.Cu") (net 1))
 (segment (start 134.55 72.45) (end 136.5 72.45) (width 0.5) (layer "B.Cu") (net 1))
 (segment (start 43 72.2) (end 44.4 72.2) (width 0.5) (layer "B.Cu") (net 1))
 (segment (start 79.4 73.35) (end 80.95 73.35) (width 0.3) (layer "F.Cu") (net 10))
 (segment (start 54.5 75) (end 77.75 75) (width 0.3) (layer "F.Cu") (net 10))
 (segment (start 51.05 76.65) (end 52.85 76.65) (width 0.3) (layer "F.Cu") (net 10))
 (segment (start 52.85 76.65) (end 54.5 75) (width 0.3) (layer "F.Cu") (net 10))
 (segment (start 77.75 75) (end 79.4 73.35) (width 0.3) (layer "F.Cu") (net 10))
 (segment (start 44.7 74.8) (end 43.7032 74.8) (width 0.2) (layer "F.Cu") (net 5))
 (segment (start 46.475 76.575) (end 44.7 74.8) (width 0.3) (layer "F.Cu") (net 5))
 (segment (start 47 76.575) (end 46.475 76.575) (width 0.3) (layer "F.Cu") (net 5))
 (segment (start 43.7032 74.8) (end 43.7 74.7968) (width 0.2) (layer "F.Cu") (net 5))
 (segment (start 78.2 76.65) (end 79.85 75) (width 0.3) (layer "F.Cu") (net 9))
 (segment (start 76.05 76.65) (end 78.2 76.65) (width 0.3) (layer "F.Cu") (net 9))
 (segment (start 104 73.35) (end 105.95 73.35) (width 0.3) (layer "F.Cu") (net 9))
 (segment (start 102.35 75) (end 104 73.35) (width 0.3) (layer "F.Cu") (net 9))
 (segment (start 79.85 75) (end 102.35 75) (width 0.3) (layer "F.Cu") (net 9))
 (segment (start 104.85 74.85) (end 127.4 74.85) (width 0.3) (layer "F.Cu") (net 8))
 (segment (start 127.4 74.85) (end 128.9 73.35) (width 0.3) (layer "F.Cu") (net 8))
 (segment (start 128.9 73.35) (end 130.95 73.35) (width 0.3) (layer "F.Cu") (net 8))
 (segment (start 103.05 76.65) (end 104.85 74.85) (width 0.3) (layer "F.Cu") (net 8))
 (segment (start 101.05 76.65) (end 103.05 76.65) (width 0.3) (layer "F.Cu") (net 8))
 (segment (start 126.05 76.65) (end 128.45 76.65) (width 0.3) (layer "F.Cu") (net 7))
 (segment (start 130.1 75) (end 135 75) (width 0.3) (layer "F.Cu") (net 7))
 (segment (start 128.45 76.65) (end 130.1 75) (width 0.3) (layer "F.Cu") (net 7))
 (segment (start 137 75) (end 137.2032 74.7968) (width 0.2) (layer "F.Cu") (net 7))
 (segment (start 137.2032 74.7968) (end 138.7 74.7968) (width 0.2) (layer "F.Cu") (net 7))
 (via (at 137 75) (size 0.6) (drill 0.3) (layers "F.Cu" "B.Cu") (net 7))
 (via (at 135 75) (size 0.6) (drill 0.3) (layers "F.Cu" "B.Cu") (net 7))
 (segment (start 135 75) (end 137 75) (width 0.3) (layer "B.Cu") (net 7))
 (segment (start 42.7 77) (end 42.7 76.1) (width 0.3) (layer "F.Cu") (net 3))
 (segment (start 133 77) (end 134 77) (width 0.3) (layer "F.Cu") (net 3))
 (segment (start 41.7865 75.1865) (end 42.5 75.9) (width 0.3) (layer "F.Cu") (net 3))
 (segment (start 42.7 76.1) (end 41.7865 75.1865) (width 0.3) (layer "F.Cu") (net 3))
 (segment (start 41.8032 75.2032) (end 42.5 75.9) (width 0.2) (layer "F.Cu") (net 3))
 (segment (start 135.7968 75.2032) (end 136.3 75.2032) (width 0.2) (layer "F.Cu") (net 3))
 (segment (start 44.05 78.35) (end 42.7 77) (width 0.3) (layer "F.Cu") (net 3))
 (segment (start 41.3 75.2032) (end 41.8032 75.2032) (width 0.2) (layer "F.Cu") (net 3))
 (segment (start 134 77) (end 135.5968 75.4032) (width 0.3) (layer "F.Cu") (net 3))
 (segment (start 133 78.2) (end 132.85 78.35) (width 0.3) (layer "F.Cu") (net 3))
 (segment (start 135.5968 75.4032) (end 135.7968 75.2032) (width 0.2) (layer "F.Cu") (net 3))
 (segment (start 132.85 78.35) (end 44.05 78.35) (width 0.3) (layer "F.Cu") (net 3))
 (via (at 133 77) (size 0.6) (drill 0.3) (layers "F.Cu" "B.Cu") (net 3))
 (via (at 133 78.2) (size 0.6) (drill 0.3) (layers "F.Cu" "B.Cu") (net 3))
 (segment (start 133 78.2) (end 133 77) (width 0.3) (layer "B.Cu") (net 3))
 (segment (start 43.7 75.2032) (end 44.1968 75.2032) (width 0.2) (layer "F.Cu") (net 6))
 (segment (start 44.2 75.2) (end 44.4 75.4) (width 0.2) (layer "F.Cu") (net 6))
 (segment (start 138.3634 75.2032) (end 138.2968 75.2032) (width 0.3) (layer "F.Cu") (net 6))
 (segment (start 137.6 77) (end 137 77.6) (width 0.3) (layer "F.Cu") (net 6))
 (segment (start 44.85 77.6) (end 44.4 77.15) (width 0.3) (layer "F.Cu") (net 6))
 (segment (start 44.4 77.15) (end 44.4 75.4) (width 0.3) (layer "F.Cu") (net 6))
 (segment (start 138.3634 75.2032) (end 138.7 75.2032) (width 0.2) (layer "F.Cu") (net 6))
 (segment (start 138.2968 75.2032) (end 137.6 75.9) (width 0.3) (layer "F.Cu") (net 6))
 (segment (start 137.6 75.9) (end 137.6 77) (width 0.3) (layer "F.Cu") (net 6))
 (segment (start 137 77.6) (end 44.85 77.6) (width 0.3) (layer "F.Cu") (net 6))
 (segment (start 44.1968 75.2032) (end 44.2 75.2) (width 0.2) (layer "F.Cu") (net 6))
 (segment (start 41.9032 74.7968) (end 41.3 74.7968) (width 0.2) (layer "F.Cu") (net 2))
 (segment (start 135.370148 72.370148) (end 135.370148 74.429852) (width 0.3) (layer "F.Cu") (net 2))
 (segment (start 135.737096 74.7968) (end 135.370148 74.429852) (width 0.2) (layer "F.Cu") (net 2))
 (segment (start 42.4 74) (end 44.6 71.8) (width 0.3) (layer "F.Cu") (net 2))
 (segment (start 42.4 74.3) (end 41.9032 74.7968) (width 0.2) (layer "F.Cu") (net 2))
 (segment (start 136.3 74.7968) (end 135.737096 74.7968) (width 0.2) (layer "F.Cu") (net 2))
 (segment (start 42.4 74.3) (end 42.4 74) (width 0.3) (layer "F.Cu") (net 2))
 (segment (start 134.8 71.8) (end 135.370148 72.370148) (width 0.3) (layer "F.Cu") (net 2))
 (segment (start 44.6 71.8) (end 134.8 71.8) (width 0.3) (layer "F.Cu") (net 2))
 (segment (start 52.209314 74.925) (end 46.75 74.925) (width 0.3) (layer "F.Cu") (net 11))
 (segment (start 55.95 73.35) (end 53.784314 73.35) (width 0.3) (layer "F.Cu") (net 11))
 (segment (start 53.784314 73.35) (end 52.209314 74.925) (width 0.3) (layer "F.Cu") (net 11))
 (segment (start 47 74.8) (end 47.2 75) (width 0.3) (layer "F.Cu") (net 11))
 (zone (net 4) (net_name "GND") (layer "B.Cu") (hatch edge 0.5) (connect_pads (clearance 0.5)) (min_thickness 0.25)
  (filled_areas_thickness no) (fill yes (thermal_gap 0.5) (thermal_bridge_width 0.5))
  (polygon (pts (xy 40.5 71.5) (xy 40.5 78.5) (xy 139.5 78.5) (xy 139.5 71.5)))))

